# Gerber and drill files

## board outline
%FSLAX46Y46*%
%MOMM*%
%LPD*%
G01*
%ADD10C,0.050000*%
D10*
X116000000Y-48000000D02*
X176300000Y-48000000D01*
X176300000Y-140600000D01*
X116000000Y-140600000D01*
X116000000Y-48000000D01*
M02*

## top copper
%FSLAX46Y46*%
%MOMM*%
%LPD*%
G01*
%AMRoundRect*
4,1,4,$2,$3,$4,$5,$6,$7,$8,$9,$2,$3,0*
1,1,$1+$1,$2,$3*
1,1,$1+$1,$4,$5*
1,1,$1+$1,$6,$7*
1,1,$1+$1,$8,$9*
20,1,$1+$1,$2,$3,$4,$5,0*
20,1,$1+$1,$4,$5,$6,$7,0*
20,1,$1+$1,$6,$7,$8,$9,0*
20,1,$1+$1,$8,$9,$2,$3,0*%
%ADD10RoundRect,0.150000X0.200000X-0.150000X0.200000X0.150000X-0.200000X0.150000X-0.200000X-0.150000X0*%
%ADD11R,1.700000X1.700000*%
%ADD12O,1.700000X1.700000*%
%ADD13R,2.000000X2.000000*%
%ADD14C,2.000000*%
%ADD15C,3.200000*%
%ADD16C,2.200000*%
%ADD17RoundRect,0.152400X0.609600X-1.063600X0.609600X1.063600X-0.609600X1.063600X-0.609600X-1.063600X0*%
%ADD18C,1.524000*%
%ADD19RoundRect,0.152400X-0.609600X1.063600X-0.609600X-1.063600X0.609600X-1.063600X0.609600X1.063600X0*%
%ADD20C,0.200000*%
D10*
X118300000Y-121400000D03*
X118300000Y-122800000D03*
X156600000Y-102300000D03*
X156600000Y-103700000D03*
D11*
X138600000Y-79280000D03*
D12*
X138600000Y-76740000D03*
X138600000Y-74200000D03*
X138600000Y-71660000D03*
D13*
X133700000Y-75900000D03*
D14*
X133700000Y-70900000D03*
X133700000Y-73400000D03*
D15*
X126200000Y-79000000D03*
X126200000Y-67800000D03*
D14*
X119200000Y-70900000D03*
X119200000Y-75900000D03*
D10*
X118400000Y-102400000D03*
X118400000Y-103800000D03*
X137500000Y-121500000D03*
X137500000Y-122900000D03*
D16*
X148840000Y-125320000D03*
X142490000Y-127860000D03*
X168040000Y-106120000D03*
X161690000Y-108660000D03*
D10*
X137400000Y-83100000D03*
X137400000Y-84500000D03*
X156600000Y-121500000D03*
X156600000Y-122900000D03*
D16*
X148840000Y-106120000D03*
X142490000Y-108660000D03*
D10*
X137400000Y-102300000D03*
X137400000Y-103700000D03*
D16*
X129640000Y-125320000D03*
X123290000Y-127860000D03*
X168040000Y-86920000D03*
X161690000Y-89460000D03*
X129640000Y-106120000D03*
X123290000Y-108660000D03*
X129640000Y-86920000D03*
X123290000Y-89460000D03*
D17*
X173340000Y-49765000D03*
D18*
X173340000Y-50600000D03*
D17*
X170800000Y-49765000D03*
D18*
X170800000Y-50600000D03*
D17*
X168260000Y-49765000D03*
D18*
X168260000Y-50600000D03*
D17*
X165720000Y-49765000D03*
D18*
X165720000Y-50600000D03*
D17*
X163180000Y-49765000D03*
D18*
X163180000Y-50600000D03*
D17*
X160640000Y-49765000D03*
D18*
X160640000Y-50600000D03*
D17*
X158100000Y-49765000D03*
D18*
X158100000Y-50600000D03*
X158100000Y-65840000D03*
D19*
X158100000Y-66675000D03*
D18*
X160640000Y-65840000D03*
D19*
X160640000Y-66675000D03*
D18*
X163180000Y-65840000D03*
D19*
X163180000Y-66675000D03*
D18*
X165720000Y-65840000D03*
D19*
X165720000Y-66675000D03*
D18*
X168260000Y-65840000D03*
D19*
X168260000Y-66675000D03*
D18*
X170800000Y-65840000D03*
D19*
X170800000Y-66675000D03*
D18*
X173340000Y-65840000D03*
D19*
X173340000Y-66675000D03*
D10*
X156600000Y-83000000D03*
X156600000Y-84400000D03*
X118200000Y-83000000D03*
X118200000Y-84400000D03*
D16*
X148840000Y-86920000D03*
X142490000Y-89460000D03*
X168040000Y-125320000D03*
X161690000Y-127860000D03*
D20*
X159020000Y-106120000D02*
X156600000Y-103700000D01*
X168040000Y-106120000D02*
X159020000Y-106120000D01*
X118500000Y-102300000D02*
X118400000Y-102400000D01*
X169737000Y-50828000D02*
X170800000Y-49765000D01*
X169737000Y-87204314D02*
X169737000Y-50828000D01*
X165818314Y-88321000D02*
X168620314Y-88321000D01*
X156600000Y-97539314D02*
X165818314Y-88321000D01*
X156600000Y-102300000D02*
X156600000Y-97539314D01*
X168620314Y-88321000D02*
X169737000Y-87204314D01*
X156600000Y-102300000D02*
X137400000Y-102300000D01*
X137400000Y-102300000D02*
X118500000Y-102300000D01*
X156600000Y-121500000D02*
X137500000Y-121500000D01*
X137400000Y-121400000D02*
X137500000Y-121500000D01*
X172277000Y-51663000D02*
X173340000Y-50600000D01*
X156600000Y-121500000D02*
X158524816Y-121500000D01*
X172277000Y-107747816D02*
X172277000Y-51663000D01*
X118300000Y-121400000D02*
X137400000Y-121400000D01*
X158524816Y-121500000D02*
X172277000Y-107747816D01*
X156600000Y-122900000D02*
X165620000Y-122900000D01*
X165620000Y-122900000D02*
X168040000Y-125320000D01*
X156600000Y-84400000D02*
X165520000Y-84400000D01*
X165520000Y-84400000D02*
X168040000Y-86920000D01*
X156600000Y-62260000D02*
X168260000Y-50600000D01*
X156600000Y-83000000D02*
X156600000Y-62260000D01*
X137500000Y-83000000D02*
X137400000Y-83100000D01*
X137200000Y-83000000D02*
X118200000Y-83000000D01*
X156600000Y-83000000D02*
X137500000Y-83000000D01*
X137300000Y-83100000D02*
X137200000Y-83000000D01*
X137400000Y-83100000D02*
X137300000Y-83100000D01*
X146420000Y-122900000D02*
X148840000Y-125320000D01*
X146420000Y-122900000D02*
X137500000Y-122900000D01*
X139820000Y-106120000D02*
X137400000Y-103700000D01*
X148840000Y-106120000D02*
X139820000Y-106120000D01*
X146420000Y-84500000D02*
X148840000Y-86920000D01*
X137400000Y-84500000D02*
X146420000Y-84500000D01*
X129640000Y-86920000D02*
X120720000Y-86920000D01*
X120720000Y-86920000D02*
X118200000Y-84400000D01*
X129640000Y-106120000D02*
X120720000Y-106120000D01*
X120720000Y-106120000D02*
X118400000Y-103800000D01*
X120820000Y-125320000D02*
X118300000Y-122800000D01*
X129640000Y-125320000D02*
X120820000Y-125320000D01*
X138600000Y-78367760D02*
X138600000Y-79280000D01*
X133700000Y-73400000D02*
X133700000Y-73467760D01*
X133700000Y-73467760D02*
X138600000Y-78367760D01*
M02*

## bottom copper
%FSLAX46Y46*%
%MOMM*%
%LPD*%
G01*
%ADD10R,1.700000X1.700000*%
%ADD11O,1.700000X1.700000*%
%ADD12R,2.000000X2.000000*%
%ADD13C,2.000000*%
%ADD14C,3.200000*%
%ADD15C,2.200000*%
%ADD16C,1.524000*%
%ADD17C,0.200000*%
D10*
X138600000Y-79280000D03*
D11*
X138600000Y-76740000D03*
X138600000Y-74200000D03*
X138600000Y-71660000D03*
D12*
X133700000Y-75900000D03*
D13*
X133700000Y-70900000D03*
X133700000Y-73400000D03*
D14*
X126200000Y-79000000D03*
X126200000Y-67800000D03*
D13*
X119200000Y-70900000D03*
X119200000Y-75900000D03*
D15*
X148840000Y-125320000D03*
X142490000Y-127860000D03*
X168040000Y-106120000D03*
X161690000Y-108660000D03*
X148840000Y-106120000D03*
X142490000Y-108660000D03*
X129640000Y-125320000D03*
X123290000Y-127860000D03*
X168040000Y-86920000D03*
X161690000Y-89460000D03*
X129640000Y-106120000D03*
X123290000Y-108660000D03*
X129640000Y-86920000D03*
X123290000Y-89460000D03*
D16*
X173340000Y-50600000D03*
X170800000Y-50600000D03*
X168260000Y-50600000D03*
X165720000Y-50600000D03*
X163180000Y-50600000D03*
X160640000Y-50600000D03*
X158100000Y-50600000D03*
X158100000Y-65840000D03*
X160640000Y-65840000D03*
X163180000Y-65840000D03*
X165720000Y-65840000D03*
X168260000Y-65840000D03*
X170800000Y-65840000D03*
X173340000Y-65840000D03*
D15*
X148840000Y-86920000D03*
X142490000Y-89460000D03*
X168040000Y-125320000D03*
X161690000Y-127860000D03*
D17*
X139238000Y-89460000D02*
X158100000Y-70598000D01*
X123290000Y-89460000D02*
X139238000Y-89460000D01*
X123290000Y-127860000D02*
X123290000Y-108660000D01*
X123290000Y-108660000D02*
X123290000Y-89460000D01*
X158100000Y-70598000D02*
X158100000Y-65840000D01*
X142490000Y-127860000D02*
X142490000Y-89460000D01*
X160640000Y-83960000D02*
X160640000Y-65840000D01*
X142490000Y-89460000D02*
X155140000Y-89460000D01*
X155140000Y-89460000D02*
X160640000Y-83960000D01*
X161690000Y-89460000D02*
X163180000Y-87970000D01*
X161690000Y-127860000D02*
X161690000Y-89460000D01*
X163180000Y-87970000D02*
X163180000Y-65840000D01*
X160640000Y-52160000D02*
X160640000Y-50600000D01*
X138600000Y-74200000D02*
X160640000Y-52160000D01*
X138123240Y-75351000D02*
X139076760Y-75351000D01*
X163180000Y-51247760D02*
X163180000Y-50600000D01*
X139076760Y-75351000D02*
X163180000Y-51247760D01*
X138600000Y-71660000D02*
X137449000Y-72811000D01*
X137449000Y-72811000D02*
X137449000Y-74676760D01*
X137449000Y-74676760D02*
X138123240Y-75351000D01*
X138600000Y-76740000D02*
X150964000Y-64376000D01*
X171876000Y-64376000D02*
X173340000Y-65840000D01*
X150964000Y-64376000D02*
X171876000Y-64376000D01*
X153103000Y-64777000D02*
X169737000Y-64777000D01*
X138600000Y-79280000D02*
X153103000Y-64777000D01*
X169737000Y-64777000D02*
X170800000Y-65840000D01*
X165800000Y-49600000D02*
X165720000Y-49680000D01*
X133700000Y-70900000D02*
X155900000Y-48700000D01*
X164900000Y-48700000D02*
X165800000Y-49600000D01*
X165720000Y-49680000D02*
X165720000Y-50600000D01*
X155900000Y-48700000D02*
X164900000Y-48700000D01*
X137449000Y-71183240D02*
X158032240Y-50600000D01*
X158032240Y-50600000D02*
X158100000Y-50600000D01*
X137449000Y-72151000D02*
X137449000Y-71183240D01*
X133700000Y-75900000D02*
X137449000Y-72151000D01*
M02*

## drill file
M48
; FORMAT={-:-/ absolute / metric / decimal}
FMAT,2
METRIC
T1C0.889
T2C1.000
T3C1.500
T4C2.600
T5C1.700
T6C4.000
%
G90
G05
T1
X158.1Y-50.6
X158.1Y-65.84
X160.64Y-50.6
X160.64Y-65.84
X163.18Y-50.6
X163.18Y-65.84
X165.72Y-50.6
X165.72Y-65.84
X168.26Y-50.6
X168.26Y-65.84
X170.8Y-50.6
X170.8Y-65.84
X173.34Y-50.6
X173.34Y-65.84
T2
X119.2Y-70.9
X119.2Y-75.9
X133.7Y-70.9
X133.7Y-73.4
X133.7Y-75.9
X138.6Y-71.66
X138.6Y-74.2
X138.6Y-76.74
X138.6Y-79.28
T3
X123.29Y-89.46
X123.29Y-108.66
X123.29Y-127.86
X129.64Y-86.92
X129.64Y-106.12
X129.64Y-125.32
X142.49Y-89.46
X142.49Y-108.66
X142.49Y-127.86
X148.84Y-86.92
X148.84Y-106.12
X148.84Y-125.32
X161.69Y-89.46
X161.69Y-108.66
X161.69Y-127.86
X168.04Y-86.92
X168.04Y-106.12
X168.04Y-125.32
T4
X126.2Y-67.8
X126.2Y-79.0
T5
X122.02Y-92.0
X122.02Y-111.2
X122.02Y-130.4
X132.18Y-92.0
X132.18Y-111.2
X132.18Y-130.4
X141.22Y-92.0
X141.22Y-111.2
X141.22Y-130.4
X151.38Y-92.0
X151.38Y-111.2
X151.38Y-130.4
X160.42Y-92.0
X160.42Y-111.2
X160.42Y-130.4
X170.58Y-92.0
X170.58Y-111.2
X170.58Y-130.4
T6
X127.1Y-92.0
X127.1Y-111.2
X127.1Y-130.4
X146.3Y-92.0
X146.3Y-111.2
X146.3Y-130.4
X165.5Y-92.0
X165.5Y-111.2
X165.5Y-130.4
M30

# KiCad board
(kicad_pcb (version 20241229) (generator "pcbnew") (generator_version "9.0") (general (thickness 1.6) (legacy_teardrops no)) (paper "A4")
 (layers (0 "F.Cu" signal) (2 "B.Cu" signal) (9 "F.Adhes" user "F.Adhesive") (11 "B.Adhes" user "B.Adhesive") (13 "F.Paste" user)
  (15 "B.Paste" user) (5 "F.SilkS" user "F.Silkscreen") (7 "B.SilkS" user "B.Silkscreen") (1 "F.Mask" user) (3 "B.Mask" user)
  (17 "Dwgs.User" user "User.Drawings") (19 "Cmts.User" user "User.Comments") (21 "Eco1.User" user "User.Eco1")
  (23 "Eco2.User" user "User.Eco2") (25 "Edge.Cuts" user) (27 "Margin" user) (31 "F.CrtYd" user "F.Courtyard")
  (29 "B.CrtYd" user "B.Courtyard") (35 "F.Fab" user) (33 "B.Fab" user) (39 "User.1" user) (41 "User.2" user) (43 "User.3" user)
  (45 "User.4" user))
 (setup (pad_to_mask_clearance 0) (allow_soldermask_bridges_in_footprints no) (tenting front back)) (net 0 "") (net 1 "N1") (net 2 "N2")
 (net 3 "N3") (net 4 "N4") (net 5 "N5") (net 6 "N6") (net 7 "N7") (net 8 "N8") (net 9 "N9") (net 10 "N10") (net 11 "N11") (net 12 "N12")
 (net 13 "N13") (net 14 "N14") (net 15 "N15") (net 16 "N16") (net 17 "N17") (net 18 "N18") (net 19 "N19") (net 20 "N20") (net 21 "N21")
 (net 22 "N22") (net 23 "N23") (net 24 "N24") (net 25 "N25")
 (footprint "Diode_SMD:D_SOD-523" (layer "F.Cu") (at 118.3 122.1 -90)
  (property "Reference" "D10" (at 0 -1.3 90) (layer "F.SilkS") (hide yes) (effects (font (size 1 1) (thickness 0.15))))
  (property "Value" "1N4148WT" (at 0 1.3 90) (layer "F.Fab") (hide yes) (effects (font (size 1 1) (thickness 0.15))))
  (pad "1" smd roundrect (at -0.7 0 90) (size 0.6 0.7) (layers "F.Cu" "F.Mask" "F.Paste") (roundrect_rratio 0.25) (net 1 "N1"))
  (pad "2" smd roundrect (at 0.7 0 90) (size 0.6 0.7) (layers "F.Cu" "F.Mask" "F.Paste") (roundrect_rratio 0.25) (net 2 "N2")))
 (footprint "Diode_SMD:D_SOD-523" (layer "F.Cu") (at 156.6 103 -90)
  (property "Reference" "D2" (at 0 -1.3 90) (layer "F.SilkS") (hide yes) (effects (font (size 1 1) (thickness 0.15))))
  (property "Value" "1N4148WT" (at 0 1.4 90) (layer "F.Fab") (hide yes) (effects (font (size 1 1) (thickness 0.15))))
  (pad "1" smd roundrect (at -0.7 0 90) (size 0.6 0.7) (layers "F.Cu" "F.Mask" "F.Paste") (roundrect_rratio 0.25) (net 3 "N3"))
  (pad "2" smd roundrect (at 0.7 0 90) (size 0.6 0.7) (layers "F.Cu" "F.Mask" "F.Paste") (roundrect_rratio 0.25) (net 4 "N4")))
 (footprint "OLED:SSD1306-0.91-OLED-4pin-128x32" (layer "F.Cu") (at 175.1 81.47 180)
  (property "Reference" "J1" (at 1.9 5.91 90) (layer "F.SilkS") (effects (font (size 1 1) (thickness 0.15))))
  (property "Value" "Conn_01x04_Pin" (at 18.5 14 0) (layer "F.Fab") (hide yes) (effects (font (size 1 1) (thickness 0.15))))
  (pad "1" thru_hole rect (at 36.5 2.19 180) (size 1.7 1.7) (drill 1) (layers "*.Cu" "*.Mask") (remove_unused_layers no) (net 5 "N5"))
  (pad "2" thru_hole oval (at 36.5 4.73 180) (size 1.7 1.7) (drill 1) (layers "*.Cu" "*.Mask") (remove_unused_layers no) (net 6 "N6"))
  (pad "3" thru_hole oval (at 36.5 7.27 180) (size 1.7 1.7) (drill 1) (layers "*.Cu" "*.Mask") (remove_unused_layers no) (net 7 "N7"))
  (pad "4" thru_hole oval (at 36.5 9.81 180) (size 1.7 1.7) (drill 1) (layers "*.Cu" "*.Mask") (remove_unused_layers no) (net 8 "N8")))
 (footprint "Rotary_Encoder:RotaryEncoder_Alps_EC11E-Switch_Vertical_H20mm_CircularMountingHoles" (layer "F.Cu") (at 133.7 75.9 180)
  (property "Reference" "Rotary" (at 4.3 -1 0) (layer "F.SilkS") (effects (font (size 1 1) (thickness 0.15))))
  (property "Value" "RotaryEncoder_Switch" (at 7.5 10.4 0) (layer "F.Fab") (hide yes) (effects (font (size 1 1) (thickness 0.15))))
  (pad "A" thru_hole rect (at 0 0 180) (size 2 2) (drill 1) (layers "*.Cu" "*.Mask") (remove_unused_layers no) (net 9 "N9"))
  (pad "B" thru_hole circle (at 0 5 180) (size 2 2) (drill 1) (layers "*.Cu" "*.Mask") (remove_unused_layers no) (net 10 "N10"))
  (pad "C" thru_hole circle (at 0 2.5 180) (size 2 2) (drill 1) (layers "*.Cu" "*.Mask") (remove_unused_layers no) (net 5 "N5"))
  (pad "MP" thru_hole circle (at 7.5 -3.1 180) (size 3.2 3.2) (drill 2.6) (layers "*.Cu" "*.Mask") (remove_unused_layers no))
  (pad "MP" thru_hole circle (at 7.5 8.1 180) (size 3.2 3.2) (drill 2.6) (layers "*.Cu" "*.Mask") (remove_unused_layers no))
  (pad "S1" thru_hole circle (at 14.5 5 180) (size 2 2) (drill 1) (layers "*.Cu" "*.Mask") (remove_unused_layers no) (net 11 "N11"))
  (pad "S2" thru_hole circle (at 14.5 0 180) (size 2 2) (drill 1) (layers "*.Cu" "*.Mask") (remove_unused_layers no) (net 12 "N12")))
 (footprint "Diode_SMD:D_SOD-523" (layer "F.Cu") (at 118.4 103.1 -90)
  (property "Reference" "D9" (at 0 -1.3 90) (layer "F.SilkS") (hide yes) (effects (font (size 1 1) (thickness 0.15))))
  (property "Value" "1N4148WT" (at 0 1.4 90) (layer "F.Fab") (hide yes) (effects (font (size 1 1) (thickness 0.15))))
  (pad "1" smd roundrect (at -0.7 0 90) (size 0.6 0.7) (layers "F.Cu" "F.Mask" "F.Paste") (roundrect_rratio 0.25) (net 3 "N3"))
  (pad "2" smd roundrect (at 0.7 0 90) (size 0.6 0.7) (layers "F.Cu" "F.Mask" "F.Paste") (roundrect_rratio 0.25) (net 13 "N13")))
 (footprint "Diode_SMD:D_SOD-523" (layer "F.Cu") (at 137.5 122.2 -90)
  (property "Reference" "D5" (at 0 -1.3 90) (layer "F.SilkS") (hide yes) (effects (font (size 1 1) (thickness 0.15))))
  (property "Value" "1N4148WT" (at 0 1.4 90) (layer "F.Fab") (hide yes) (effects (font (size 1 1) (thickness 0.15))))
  (pad "1" smd roundrect (at -0.7 0 90) (size 0.6 0.7) (layers "F.Cu" "F.Mask" "F.Paste") (roundrect_rratio 0.25) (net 1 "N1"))
  (pad "2" smd roundrect (at 0.7 0 90) (size 0.6 0.7) (layers "F.Cu" "F.Mask" "F.Paste") (roundrect_rratio 0.25) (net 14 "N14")))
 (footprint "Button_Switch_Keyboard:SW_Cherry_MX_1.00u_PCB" (layer "F.Cu") (at 148.84 125.32)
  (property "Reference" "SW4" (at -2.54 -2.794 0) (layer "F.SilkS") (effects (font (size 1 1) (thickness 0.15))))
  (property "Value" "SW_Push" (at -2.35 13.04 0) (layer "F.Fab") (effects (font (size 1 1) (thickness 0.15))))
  (pad "" np_thru_hole circle (at -7.62 5.08) (size 1.7 1.7) (drill 1.7) (layers "*.Cu" "*.Mask"))
  (pad "" np_thru_hole circle (at -2.54 5.08) (size 4 4) (drill 4) (layers "*.Cu" "*.Mask"))
  (pad "" np_thru_hole circle (at 2.54 5.08) (size 1.7 1.7) (drill 1.7) (layers "*.Cu" "*.Mask"))
  (pad "1" thru_hole circle (at 0 0) (size 2.2 2.2) (drill 1.5) (layers "*.Cu" "*.Mask") (remove_unused_layers no) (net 14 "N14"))
  (pad "2" thru_hole circle (at -6.35 2.54) (size 2.2 2.2) (drill 1.5) (layers "*.Cu" "*.Mask") (remove_unused_layers no) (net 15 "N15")))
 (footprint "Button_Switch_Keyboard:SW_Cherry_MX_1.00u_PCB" (layer "F.Cu") (at 168.04 106.12)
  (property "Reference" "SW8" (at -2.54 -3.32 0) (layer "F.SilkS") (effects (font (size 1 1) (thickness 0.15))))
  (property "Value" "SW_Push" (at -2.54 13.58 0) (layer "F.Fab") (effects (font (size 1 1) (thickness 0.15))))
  (pad "" np_thru_hole circle (at -7.62 5.08) (size 1.7 1.7) (drill 1.7) (layers "*.Cu" "*.Mask"))
  (pad "" np_thru_hole circle (at -2.54 5.08) (size 4 4) (drill 4) (layers "*.Cu" "*.Mask"))
  (pad "" np_thru_hole circle (at 2.54 5.08) (size 1.7 1.7) (drill 1.7) (layers "*.Cu" "*.Mask"))
  (pad "1" thru_hole circle (at 0 0) (size 2.2 2.2) (drill 1.5) (layers "*.Cu" "*.Mask") (remove_unused_layers no) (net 4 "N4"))
  (pad "2" thru_hole circle (at -6.35 2.54) (size 2.2 2.2) (drill 1.5) (layers "*.Cu" "*.Mask") (remove_unused_layers no) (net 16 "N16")))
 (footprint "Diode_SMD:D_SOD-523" (layer "F.Cu") (at 137.4 83.8 -90)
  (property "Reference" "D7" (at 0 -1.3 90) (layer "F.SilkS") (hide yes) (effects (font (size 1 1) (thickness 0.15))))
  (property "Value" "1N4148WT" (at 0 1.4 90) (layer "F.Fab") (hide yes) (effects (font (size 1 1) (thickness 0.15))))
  (pad "1" smd roundrect (at -0.7 0 90) (size 0.6 0.7) (layers "F.Cu" "F.Mask" "F.Paste") (roundrect_rratio 0.25) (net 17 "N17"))
  (pad "2" smd roundrect (at 0.7 0 90) (size 0.6 0.7) (layers "F.Cu" "F.Mask" "F.Paste") (roundrect_rratio 0.25) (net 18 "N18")))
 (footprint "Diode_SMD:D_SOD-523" (layer "F.Cu") (at 156.6 122.2 -90)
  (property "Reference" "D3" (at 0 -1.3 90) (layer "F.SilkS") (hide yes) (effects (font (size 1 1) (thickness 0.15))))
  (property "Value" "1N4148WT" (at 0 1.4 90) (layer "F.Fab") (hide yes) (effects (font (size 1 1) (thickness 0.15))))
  (pad "1" smd roundrect (at -0.7 0 90) (size 0.6 0.7) (layers "F.Cu" "F.Mask" "F.Paste") (roundrect_rratio 0.25) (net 1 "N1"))
  (pad "2" smd roundrect (at 0.7 0 90) (size 0.6 0.7) (layers "F.Cu" "F.Mask" "F.Paste") (roundrect_rratio 0.25) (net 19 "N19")))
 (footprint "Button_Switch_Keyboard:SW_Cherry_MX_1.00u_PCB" (layer "F.Cu") (at 148.84 106.12)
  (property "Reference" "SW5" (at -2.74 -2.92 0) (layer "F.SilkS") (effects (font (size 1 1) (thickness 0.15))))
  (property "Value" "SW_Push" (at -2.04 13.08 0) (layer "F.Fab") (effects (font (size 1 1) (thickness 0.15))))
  (pad "" np_thru_hole circle (at -7.62 5.08) (size 1.7 1.7) (drill 1.7) (layers "*.Cu" "*.Mask"))
  (pad "" np_thru_hole circle (at -2.54 5.08) (size 4 4) (drill 4) (layers "*.Cu" "*.Mask"))
  (pad "" np_thru_hole circle (at 2.54 5.08) (size 1.7 1.7) (drill 1.7) (layers "*.Cu" "*.Mask"))
  (pad "1" thru_hole circle (at 0 0) (size 2.2 2.2) (drill 1.5) (layers "*.Cu" "*.Mask") (remove_unused_layers no) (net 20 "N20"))
  (pad "2" thru_hole circle (at -6.35 2.54) (size 2.2 2.2) (drill 1.5) (layers "*.Cu" "*.Mask") (remove_unused_layers no) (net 15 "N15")))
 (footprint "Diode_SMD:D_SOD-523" (layer "F.Cu") (at 137.4 103 -90)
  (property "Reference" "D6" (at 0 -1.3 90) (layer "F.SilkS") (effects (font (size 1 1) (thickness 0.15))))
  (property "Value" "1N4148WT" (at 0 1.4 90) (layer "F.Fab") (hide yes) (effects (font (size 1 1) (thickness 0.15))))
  (pad "1" smd roundrect (at -0.7 0 90) (size 0.6 0.7) (layers "F.Cu" "F.Mask" "F.Paste") (roundrect_rratio 0.25) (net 3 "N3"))
  (pad "2" smd roundrect (at 0.7 0 90) (size 0.6 0.7) (layers "F.Cu" "F.Mask" "F.Paste") (roundrect_rratio 0.25) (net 20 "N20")))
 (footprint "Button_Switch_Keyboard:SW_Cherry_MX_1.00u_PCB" (layer "F.Cu") (at 129.64 125.32)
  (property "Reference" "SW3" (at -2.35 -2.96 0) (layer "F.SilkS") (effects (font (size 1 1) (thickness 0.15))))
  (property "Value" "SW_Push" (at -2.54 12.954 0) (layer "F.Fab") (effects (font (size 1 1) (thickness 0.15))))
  (pad "" np_thru_hole circle (at -7.62 5.08) (size 1.7 1.7) (drill 1.7) (layers "*.Cu" "*.Mask"))
  (pad "" np_thru_hole circle (at -2.54 5.08) (size 4 4) (drill 4) (layers "*.Cu" "*.Mask"))
  (pad "" np_thru_hole circle (at 2.54 5.08) (size 1.7 1.7) (drill 1.7) (layers "*.Cu" "*.Mask"))
  (pad "1" thru_hole circle (at 0 0) (size 2.2 2.2) (drill 1.5) (layers "*.Cu" "*.Mask") (remove_unused_layers no) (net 2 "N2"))
  (pad "2" thru_hole circle (at -6.35 2.54) (size 2.2 2.2) (drill 1.5) (layers "*.Cu" "*.Mask") (remove_unused_layers no) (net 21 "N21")))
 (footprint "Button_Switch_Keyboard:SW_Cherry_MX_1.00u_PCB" (layer "F.Cu") (at 168.04 86.92)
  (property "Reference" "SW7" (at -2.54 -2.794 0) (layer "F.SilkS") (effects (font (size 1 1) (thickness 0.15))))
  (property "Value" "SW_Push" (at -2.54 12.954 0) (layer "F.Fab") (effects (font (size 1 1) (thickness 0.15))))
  (pad "" np_thru_hole circle (at -7.62 5.08) (size 1.7 1.7) (drill 1.7) (layers "*.Cu" "*.Mask"))
  (pad "" np_thru_hole circle (at -2.54 5.08) (size 4 4) (drill 4) (layers "*.Cu" "*.Mask"))
  (pad "" np_thru_hole circle (at 2.54 5.08) (size 1.7 1.7) (drill 1.7) (layers "*.Cu" "*.Mask"))
  (pad "1" thru_hole circle (at 0 0) (size 2.2 2.2) (drill 1.5) (layers "*.Cu" "*.Mask") (remove_unused_layers no) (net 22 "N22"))
  (pad "2" thru_hole circle (at -6.35 2.54) (size 2.2 2.2) (drill 1.5) (layers "*.Cu" "*.Mask") (remove_unused_layers no) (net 16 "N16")))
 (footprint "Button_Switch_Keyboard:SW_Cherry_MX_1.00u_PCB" (layer "F.Cu") (at 129.64 106.12)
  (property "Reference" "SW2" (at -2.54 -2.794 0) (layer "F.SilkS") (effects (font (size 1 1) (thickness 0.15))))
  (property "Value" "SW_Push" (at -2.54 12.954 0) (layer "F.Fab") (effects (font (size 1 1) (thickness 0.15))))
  (pad "" np_thru_hole circle (at -7.62 5.08) (size 1.7 1.7) (drill 1.7) (layers "*.Cu" "*.Mask"))
  (pad "" np_thru_hole circle (at -2.54 5.08) (size 4 4) (drill 4) (layers "*.Cu" "*.Mask"))
  (pad "" np_thru_hole circle (at 2.54 5.08) (size 1.7 1.7) (drill 1.7) (layers "*.Cu" "*.Mask"))
  (pad "1" thru_hole circle (at 0 0) (size 2.2 2.2) (drill 1.5) (layers "*.Cu" "*.Mask") (remove_unused_layers no) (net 13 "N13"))
  (pad "2" thru_hole circle (at -6.35 2.54) (size 2.2 2.2) (drill 1.5) (layers "*.Cu" "*.Mask") (remove_unused_layers no) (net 21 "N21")))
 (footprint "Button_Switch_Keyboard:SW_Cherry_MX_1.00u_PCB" (layer "F.Cu") (at 129.64 86.92)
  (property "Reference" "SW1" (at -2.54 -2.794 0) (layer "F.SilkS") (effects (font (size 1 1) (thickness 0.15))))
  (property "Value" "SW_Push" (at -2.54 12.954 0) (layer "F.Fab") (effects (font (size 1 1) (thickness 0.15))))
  (pad "" np_thru_hole circle (at -7.62 5.08) (size 1.7 1.7) (drill 1.7) (layers "*.Cu" "*.Mask"))
  (pad "" np_thru_hole circle (at -2.54 5.08) (size 4 4) (drill 4) (layers "*.Cu" "*.Mask"))
  (pad "" np_thru_hole circle (at 2.54 5.08) (size 1.7 1.7) (drill 1.7) (layers "*.Cu" "*.Mask"))
  (pad "1" thru_hole circle (at 0 0) (size 2.2 2.2) (drill 1.5) (layers "*.Cu" "*.Mask") (remove_unused_layers no) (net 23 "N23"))
  (pad "2" thru_hole circle (at -6.35 2.54) (size 2.2 2.2) (drill 1.5) (layers "*.Cu" "*.Mask") (remove_unused_layers no) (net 21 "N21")))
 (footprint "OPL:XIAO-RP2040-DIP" (layer "F.Cu") (at 165.72 58.22 -90)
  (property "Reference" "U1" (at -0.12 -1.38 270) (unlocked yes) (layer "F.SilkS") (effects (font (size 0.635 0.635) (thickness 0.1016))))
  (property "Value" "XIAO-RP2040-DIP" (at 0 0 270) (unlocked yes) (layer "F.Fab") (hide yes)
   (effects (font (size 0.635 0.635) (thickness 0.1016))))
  (pad "1" smd roundrect (at -8.455 -7.62 90) (size 2.432 1.524) (layers "F.Cu" "F.Mask") (roundrect_rratio 0.1) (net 1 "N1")
   (thermal_bridge_angle 45))
  (pad "1" thru_hole circle (at -7.62 -7.62 90) (size 1.524 1.524) (drill 0.889) (layers "*.Cu" "*.Mask") (remove_unused_layers no)
   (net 1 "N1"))
  (pad "2" smd roundrect (at -8.455 -5.08 90) (size 2.432 1.524) (layers "F.Cu" "F.Mask") (roundrect_rratio 0.1) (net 3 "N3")
   (thermal_bridge_angle 45))
  (pad "2" thru_hole circle (at -7.62 -5.08 90) (size 1.524 1.524) (drill 0.889) (layers "*.Cu" "*.Mask") (remove_unused_layers no)
   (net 3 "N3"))
  (pad "3" smd roundrect (at -8.455 -2.54 90) (size 2.432 1.524) (layers "F.Cu" "F.Mask") (roundrect_rratio 0.1) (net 17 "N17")
   (thermal_bridge_angle 45))
  (pad "3" thru_hole circle (at -7.62 -2.54 90) (size 1.524 1.524) (drill 0.889) (layers "*.Cu" "*.Mask") (remove_unused_layers no)
   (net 17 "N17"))
  (pad "4" smd roundrect (at -8.455 0 90) (size 2.432 1.524) (layers "F.Cu" "F.Mask") (roundrect_rratio 0.1) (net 10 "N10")
   (thermal_bridge_angle 45))
  (pad "4" thru_hole circle (at -7.62 0 90) (size 1.524 1.524) (drill 0.889) (layers "*.Cu" "*.Mask") (remove_unused_layers no)
   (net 10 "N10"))
  (pad "5" smd roundrect (at -8.455 2.54 90) (size 2.432 1.524) (layers "F.Cu" "F.Mask") (roundrect_rratio 0.1) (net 8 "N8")
   (thermal_bridge_angle 45))
  (pad "5" thru_hole circle (at -7.62 2.54 90) (size 1.524 1.524) (drill 0.889) (layers "*.Cu" "*.Mask") (remove_unused_layers no)
   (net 8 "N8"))
  (pad "6" smd roundrect (at -8.455 5.08 90) (size 2.432 1.524) (layers "F.Cu" "F.Mask") (roundrect_rratio 0.1) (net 7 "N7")
   (thermal_bridge_angle 45))
  (pad "6" thru_hole circle (at -7.62 5.08 90) (size 1.524 1.524) (drill 0.889) (layers "*.Cu" "*.Mask") (remove_unused_layers no)
   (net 7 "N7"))
  (pad "7" smd roundrect (at -8.455 7.62 90) (size 2.432 1.524) (layers "F.Cu" "F.Mask") (roundrect_rratio 0.1) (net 9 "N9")
   (thermal_bridge_angle 45))
  (pad "7" thru_hole circle (at -7.62 7.62 90) (size 1.524 1.524) (drill 0.889) (layers "*.Cu" "*.Mask") (remove_unused_layers no)
   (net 9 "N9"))
  (pad "8" thru_hole circle (at 7.62 7.62 270) (size 1.524 1.524) (drill 0.889) (layers "*.Cu" "*.Mask") (remove_unused_layers no)
   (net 21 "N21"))
  (pad "8" smd roundrect (at 8.455 7.62 270) (size 2.432 1.524) (layers "F.Cu" "F.Mask") (roundrect_rratio 0.1) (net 21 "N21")
   (thermal_bridge_angle 45))
  (pad "9" thru_hole circle (at 7.62 5.08 270) (size 1.524 1.524) (drill 0.889) (layers "*.Cu" "*.Mask") (remove_unused_layers no)
   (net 15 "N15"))
  (pad "9" smd roundrect (at 8.455 5.08 270) (size 2.432 1.524) (layers "F.Cu" "F.Mask") (roundrect_rratio 0.1) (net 15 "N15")
   (thermal_bridge_angle 45))
  (pad "10" thru_hole circle (at 7.62 2.54 270) (size 1.524 1.524) (drill 0.889) (layers "*.Cu" "*.Mask") (remove_unused_layers no)
   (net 16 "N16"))
  (pad "10" smd roundrect (at 8.455 2.54 270) (size 2.432 1.524) (layers "F.Cu" "F.Mask") (roundrect_rratio 0.1) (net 16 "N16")
   (thermal_bridge_angle 45))
  (pad "11" thru_hole circle (at 7.62 0 270) (size 1.524 1.524) (drill 0.889) (layers "*.Cu" "*.Mask") (remove_unused_layers no)
   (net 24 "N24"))
  (pad "11" smd roundrect (at 8.455 0 270) (size 2.432 1.524) (layers "F.Cu" "F.Mask") (roundrect_rratio 0.1) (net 24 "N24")
   (thermal_bridge_angle 45))
  (pad "12" thru_hole circle (at 7.62 -2.54 270) (size 1.524 1.524) (drill 0.889) (layers "*.Cu" "*.Mask") (remove_unused_layers no)
   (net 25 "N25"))
  (pad "12" smd roundrect (at 8.455 -2.54 270) (size 2.432 1.524) (layers "F.Cu" "F.Mask") (roundrect_rratio 0.1) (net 25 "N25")
   (thermal_bridge_angle 45))
  (pad "13" thru_hole circle (at 7.62 -5.08 270) (size 1.524 1.524) (drill 0.889) (layers "*.Cu" "*.Mask") (remove_unused_layers no)
   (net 5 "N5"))
  (pad "13" smd roundrect (at 8.455 -5.08 270) (size 2.432 1.524) (layers "F.Cu" "F.Mask") (roundrect_rratio 0.1) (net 5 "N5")
   (thermal_bridge_angle 45))
  (pad "14" thru_hole circle (at 7.62 -7.62 270) (size 1.524 1.524) (drill 0.889) (layers "*.Cu" "*.Mask") (remove_unused_layers no)
   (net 6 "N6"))
  (pad "14" smd roundrect (at 8.455 -7.62 270) (size 2.432 1.524) (layers "F.Cu" "F.Mask") (roundrect_rratio 0.1) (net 6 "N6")
   (thermal_bridge_angle 45)))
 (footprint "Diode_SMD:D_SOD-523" (layer "F.Cu") (at 156.6 83.7 -90)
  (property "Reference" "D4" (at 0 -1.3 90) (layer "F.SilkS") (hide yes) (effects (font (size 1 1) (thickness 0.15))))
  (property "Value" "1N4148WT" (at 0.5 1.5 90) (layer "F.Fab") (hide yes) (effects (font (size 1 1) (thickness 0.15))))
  (pad "1" smd roundrect (at -0.7 0 90) (size 0.6 0.7) (layers "F.Cu" "F.Mask" "F.Paste") (roundrect_rratio 0.25) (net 17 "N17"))
  (pad "2" smd roundrect (at 0.7 0 90) (size 0.6 0.7) (layers "F.Cu" "F.Mask" "F.Paste") (roundrect_rratio 0.25) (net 22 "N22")))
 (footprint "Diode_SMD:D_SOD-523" (layer "F.Cu") (at 118.2 83.7 -90)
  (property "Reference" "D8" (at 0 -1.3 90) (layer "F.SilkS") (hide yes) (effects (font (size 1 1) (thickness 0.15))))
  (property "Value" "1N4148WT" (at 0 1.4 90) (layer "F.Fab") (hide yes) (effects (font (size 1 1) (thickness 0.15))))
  (pad "1" smd roundrect (at -0.7 0 90) (size 0.6 0.7) (layers "F.Cu" "F.Mask" "F.Paste") (roundrect_rratio 0.25) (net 17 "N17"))
  (pad "2" smd roundrect (at 0.7 0 90) (size 0.6 0.7) (layers "F.Cu" "F.Mask" "F.Paste") (roundrect_rratio 0.25) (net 23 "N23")))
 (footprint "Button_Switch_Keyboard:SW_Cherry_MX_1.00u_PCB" (layer "F.Cu") (at 148.84 86.92)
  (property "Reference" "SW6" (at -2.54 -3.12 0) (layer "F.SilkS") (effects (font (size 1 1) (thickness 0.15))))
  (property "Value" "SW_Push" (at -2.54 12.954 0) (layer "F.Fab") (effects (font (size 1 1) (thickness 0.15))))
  (pad "" np_thru_hole circle (at -7.62 5.08) (size 1.7 1.7) (drill 1.7) (layers "*.Cu" "*.Mask"))
  (pad "" np_thru_hole circle (at -2.54 5.08) (size 4 4) (drill 4) (layers "*.Cu" "*.Mask"))
  (pad "" np_thru_hole circle (at 2.54 5.08) (size 1.7 1.7) (drill 1.7) (layers "*.Cu" "*.Mask"))
  (pad "1" thru_hole circle (at 0 0) (size 2.2 2.2) (drill 1.5) (layers "*.Cu" "*.Mask") (remove_unused_layers no) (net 18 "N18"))
  (pad "2" thru_hole circle (at -6.35 2.54) (size 2.2 2.2) (drill 1.5) (layers "*.Cu" "*.Mask") (remove_unused_layers no) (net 15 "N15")))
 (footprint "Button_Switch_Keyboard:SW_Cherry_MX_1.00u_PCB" (layer "F.Cu") (at 168.04 125.32)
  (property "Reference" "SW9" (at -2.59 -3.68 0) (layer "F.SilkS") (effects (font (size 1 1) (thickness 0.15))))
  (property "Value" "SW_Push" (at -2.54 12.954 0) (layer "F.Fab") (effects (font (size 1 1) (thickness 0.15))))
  (pad "" np_thru_hole circle (at -7.62 5.08) (size 1.7 1.7) (drill 1.7) (layers "*.Cu" "*.Mask"))
  (pad "" np_thru_hole circle (at -2.54 5.08) (size 4 4) (drill 4) (layers "*.Cu" "*.Mask"))
  (pad "" np_thru_hole circle (at 2.54 5.08) (size 1.7 1.7) (drill 1.7) (layers "*.Cu" "*.Mask"))
  (pad "1" thru_hole circle (at 0 0) (size 2.2 2.2) (drill 1.5) (layers "*.Cu" "*.Mask") (remove_unused_layers no) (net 19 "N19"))
  (pad "2" thru_hole circle (at -6.35 2.54) (size 2.2 2.2) (drill 1.5) (layers "*.Cu" "*.Mask") (remove_unused_layers no) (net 16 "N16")))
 (gr_rect (start 116 48) (end 176.3 140.6) (stroke (width 0.05) (type default)) (fill no) (layer "Edge.Cuts"))
 (segment (start 159.02 106.12) (end 156.6 103.7) (width 0.2) (layer "F.Cu") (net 4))
 (segment (start 168.04 106.12) (end 159.02 106.12) (width 0.2) (layer "F.Cu") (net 4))
 (segment (start 118.5 102.3) (end 118.4 102.4) (width 0.2) (layer "F.Cu") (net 3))
 (segment (start 169.737 50.828) (end 170.8 49.765) (width 0.2) (layer "F.Cu") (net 3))
 (segment (start 169.737 87.204314) (end 169.737 50.828) (width 0.2) (layer "F.Cu") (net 3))
 (segment (start 165.818314 88.321) (end 168.620314 88.321) (width 0.2) (layer "F.Cu") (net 3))
 (segment (start 156.6 97.539314) (end 165.818314 88.321) (width 0.2) (layer "F.Cu") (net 3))
 (segment (start 156.6 102.3) (end 156.6 97.539314) (width 0.2) (layer "F.Cu") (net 3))
 (segment (start 168.620314 88.321) (end 169.737 87.204314) (width 0.2) (layer "F.Cu") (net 3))
 (segment (start 156.6 102.3) (end 137.4 102.3) (width 0.2) (layer "F.Cu") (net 3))
 (segment (start 137.4 102.3) (end 118.5 102.3) (width 0.2) (layer "F.Cu") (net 3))
 (segment (start 156.6 121.5) (end 137.5 121.5) (width 0.2) (layer "F.Cu") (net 1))
 (segment (start 137.4 121.4) (end 137.5 121.5) (width 0.2) (layer "F.Cu") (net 1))
 (segment (start 172.277 51.663) (end 173.34 50.6) (width 0.2) (layer "F.Cu") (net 1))
 (segment (start 156.6 121.5) (end 158.524816 121.5) (width 0.2) (layer "F.Cu") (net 1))
 (segment (start 172.277 107.747816) (end 172.277 51.663) (width 0.2) (layer "F.Cu") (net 1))
 (segment (start 118.3 121.4) (end 137.4 121.4) (width 0.2) (layer "F.Cu") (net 1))
 (segment (start 158.524816 121.5) (end 172.277 107.747816) (width 0.2) (layer "F.Cu") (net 1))
 (segment (start 156.6 122.9) (end 165.62 122.9) (width 0.2) (layer "F.Cu") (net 19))
 (segment (start 165.62 122.9) (end 168.04 125.32) (width 0.2) (layer "F.Cu") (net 19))
 (segment (start 156.6 84.4) (end 165.52 84.4) (width 0.2) (layer "F.Cu") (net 22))
 (segment (start 165.52 84.4) (end 168.04 86.92) (width 0.2) (layer "F.Cu") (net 22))
 (segment (start 156.6 62.26) (end 168.26 50.6) (width 0.2) (layer "F.Cu") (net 17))
 (segment (start 156.6 83) (end 156.6 62.26) (width 0.2) (layer "F.Cu") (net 17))
 (segment (start 137.5 83) (end 137.4 83.1) (width 0.2) (layer "F.Cu") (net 17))
 (segment (start 137.2 83) (end 118.2 83) (width 0.2) (layer "F.Cu") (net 17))
 (segment (start 156.6 83) (end 137.5 83) (width 0.2) (layer "F.Cu") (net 17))
 (segment (start 137.3 83.1) (end 137.2 83) (width 0.2) (layer "F.Cu") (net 17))
 (segment (start 137.4 83.1) (end 137.3 83.1) (width 0.2) (layer "F.Cu") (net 17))
 (segment (start 146.42 122.9) (end 148.84 125.32) (width 0.2) (layer "F.Cu") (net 14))
 (segment (start 146.42 122.9) (end 137.5 122.9) (width 0.2) (layer "F.Cu") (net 14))
 (segment (start 139.82 106.12) (end 137.4 103.7) (width 0.2) (layer "F.Cu") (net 20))
 (segment (start 148.84 106.12) (end 139.82 106.12) (width 0.2) (layer "F.Cu") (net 20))
 (segment (start 146.42 84.5) (end 148.84 86.92) (width 0.2) (layer "F.Cu") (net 18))
 (segment (start 137.4 84.5) (end 146.42 84.5) (width 0.2) (layer "F.Cu") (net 18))
 (segment (start 129.64 86.92) (end 120.72 86.92) (width 0.2) (layer "F.Cu") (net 23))
 (segment (start 120.72 86.92) (end 118.2 84.4) (width 0.2) (layer "F.Cu") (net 23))
 (segment (start 129.64 106.12) (end 120.72 106.12) (width 0.2) (layer "F.Cu") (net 13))
 (segment (start 120.72 106.12) (end 118.4 103.8) (width 0.2) (layer "F.Cu") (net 13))
 (segment (start 120.82 125.32) (end 118.3 122.8) (width 0.2) (layer "F.Cu") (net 2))
 (segment (start 129.64 125.32) (end 120.82 125.32) (width 0.2) (layer "F.Cu") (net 2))
 (segment (start 139.238 89.46) (end 158.1 70.598) (width 0.2) (layer "B.Cu") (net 21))
 (segment (start 123.29 89.46) (end 139.238 89.46) (width 0.2) (layer "B.Cu") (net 21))
 (segment (start 123.29 127.86) (end 123.29 108.66) (width 0.2) (layer "B.Cu") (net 21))
 (segment (start 123.29 108.66) (end 123.29 89.46) (width 0.2) (layer "B.Cu") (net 21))
 (segment (start 158.1 70.598) (end 158.1 65.84) (width 0.2) (layer "B.Cu") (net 21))
 (segment (start 142.49 127.86) (end 142.49 89.46) (width 0.2) (layer "B.Cu") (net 15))
 (segment (start 160.64 83.96) (end 160.64 65.84) (width 0.2) (layer "B.Cu") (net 15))
 (segment (start 142.49 89.46) (end 155.14 89.46) (width 0.2) (layer "B.Cu") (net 15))
 (segment (start 155.14 89.46) (end 160.64 83.96) (width 0.2) (layer "B.Cu") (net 15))
 (segment (start 161.69 89.46) (end 163.18 87.97) (width 0.2) (layer "B.Cu") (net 16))
 (segment (start 161.69 127.86) (end 161.69 89.46) (width 0.2) (layer "B.Cu") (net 16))
 (segment (start 163.18 87.97) (end 163.18 65.84) (width 0.2) (layer "B.Cu") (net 16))
 (segment (start 160.64 52.16) (end 160.64 50.6) (width 0.2) (layer "B.Cu") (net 7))
 (segment (start 138.6 74.2) (end 160.64 52.16) (width 0.2) (layer "B.Cu") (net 7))
 (segment (start 138.12324 75.351) (end 139.07676 75.351) (width 0.2) (layer "B.Cu") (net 8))
 (segment (start 163.18 51.24776) (end 163.18 50.6) (width 0.2) (layer "B.Cu") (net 8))
 (segment (start 139.07676 75.351) (end 163.18 51.24776) (width 0.2) (layer "B.Cu") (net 8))
 (segment (start 138.6 71.66) (end 137.449 72.811) (width 0.2) (layer "B.Cu") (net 8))
 (segment (start 137.449 72.811) (end 137.449 74.67676) (width 0.2) (layer "B.Cu") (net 8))
 (segment (start 137.449 74.67676) (end 138.12324 75.351) (width 0.2) (layer "B.Cu") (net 8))
 (segment (start 138.6 76.74) (end 150.964 64.376) (width 0.2) (layer "B.Cu") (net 6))
 (segment (start 171.876 64.376) (end 173.34 65.84) (width 0.2) (layer "B.Cu") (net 6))
 (segment (start 150.964 64.376) (end 171.876 64.376) (width 0.2) (layer "B.Cu") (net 6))
 (segment (start 138.6 78.36776) (end 138.6 79.28) (width 0.2) (layer "F.Cu") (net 5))
 (segment (start 133.7 73.4) (end 133.7 73.46776) (width 0.2) (layer "F.Cu") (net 5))
 (segment (start 133.7 73.46776) (end 138.6 78.36776) (width 0.2) (layer "F.Cu") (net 5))
 (segment (start 153.103 64.777) (end 169.737 64.777) (width 0.2) (layer "B.Cu") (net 5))
 (segment (start 138.6 79.28) (end 153.103 64.777) (width 0.2) (layer "B.Cu") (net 5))
 (segment (start 169.737 64.777) (end 170.8 65.84) (width 0.2) (layer "B.Cu") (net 5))
 (segment (start 165.8 49.6) (end 165.72 49.68) (width 0.2) (layer "B.Cu") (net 10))
 (segment (start 133.7 70.9) (end 155.9 48.7) (width 0.2) (layer "B.Cu") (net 10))
 (segment (start 164.9 48.7) (end 165.8 49.6) (width 0.2) (layer "B.Cu") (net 10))
 (segment (start 165.72 49.68) (end 165.72 50.6) (width 0.2) (layer "B.Cu") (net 10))
 (segment (start 155.9 48.7) (end 164.9 48.7) (width 0.2) (layer "B.Cu") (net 10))
 (segment (start 137.449 71.18324) (end 158.03224 50.6) (width 0.2) (layer "B.Cu") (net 9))
 (segment (start 158.03224 50.6) (end 158.1 50.6) (width 0.2) (layer "B.Cu") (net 9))
 (segment (start 137.449 72.151) (end 137.449 71.18324) (width 0.2) (layer "B.Cu") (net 9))
 (segment (start 133.7 75.9) (end 137.449 72.151) (width 0.2) (layer "B.Cu") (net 9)))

